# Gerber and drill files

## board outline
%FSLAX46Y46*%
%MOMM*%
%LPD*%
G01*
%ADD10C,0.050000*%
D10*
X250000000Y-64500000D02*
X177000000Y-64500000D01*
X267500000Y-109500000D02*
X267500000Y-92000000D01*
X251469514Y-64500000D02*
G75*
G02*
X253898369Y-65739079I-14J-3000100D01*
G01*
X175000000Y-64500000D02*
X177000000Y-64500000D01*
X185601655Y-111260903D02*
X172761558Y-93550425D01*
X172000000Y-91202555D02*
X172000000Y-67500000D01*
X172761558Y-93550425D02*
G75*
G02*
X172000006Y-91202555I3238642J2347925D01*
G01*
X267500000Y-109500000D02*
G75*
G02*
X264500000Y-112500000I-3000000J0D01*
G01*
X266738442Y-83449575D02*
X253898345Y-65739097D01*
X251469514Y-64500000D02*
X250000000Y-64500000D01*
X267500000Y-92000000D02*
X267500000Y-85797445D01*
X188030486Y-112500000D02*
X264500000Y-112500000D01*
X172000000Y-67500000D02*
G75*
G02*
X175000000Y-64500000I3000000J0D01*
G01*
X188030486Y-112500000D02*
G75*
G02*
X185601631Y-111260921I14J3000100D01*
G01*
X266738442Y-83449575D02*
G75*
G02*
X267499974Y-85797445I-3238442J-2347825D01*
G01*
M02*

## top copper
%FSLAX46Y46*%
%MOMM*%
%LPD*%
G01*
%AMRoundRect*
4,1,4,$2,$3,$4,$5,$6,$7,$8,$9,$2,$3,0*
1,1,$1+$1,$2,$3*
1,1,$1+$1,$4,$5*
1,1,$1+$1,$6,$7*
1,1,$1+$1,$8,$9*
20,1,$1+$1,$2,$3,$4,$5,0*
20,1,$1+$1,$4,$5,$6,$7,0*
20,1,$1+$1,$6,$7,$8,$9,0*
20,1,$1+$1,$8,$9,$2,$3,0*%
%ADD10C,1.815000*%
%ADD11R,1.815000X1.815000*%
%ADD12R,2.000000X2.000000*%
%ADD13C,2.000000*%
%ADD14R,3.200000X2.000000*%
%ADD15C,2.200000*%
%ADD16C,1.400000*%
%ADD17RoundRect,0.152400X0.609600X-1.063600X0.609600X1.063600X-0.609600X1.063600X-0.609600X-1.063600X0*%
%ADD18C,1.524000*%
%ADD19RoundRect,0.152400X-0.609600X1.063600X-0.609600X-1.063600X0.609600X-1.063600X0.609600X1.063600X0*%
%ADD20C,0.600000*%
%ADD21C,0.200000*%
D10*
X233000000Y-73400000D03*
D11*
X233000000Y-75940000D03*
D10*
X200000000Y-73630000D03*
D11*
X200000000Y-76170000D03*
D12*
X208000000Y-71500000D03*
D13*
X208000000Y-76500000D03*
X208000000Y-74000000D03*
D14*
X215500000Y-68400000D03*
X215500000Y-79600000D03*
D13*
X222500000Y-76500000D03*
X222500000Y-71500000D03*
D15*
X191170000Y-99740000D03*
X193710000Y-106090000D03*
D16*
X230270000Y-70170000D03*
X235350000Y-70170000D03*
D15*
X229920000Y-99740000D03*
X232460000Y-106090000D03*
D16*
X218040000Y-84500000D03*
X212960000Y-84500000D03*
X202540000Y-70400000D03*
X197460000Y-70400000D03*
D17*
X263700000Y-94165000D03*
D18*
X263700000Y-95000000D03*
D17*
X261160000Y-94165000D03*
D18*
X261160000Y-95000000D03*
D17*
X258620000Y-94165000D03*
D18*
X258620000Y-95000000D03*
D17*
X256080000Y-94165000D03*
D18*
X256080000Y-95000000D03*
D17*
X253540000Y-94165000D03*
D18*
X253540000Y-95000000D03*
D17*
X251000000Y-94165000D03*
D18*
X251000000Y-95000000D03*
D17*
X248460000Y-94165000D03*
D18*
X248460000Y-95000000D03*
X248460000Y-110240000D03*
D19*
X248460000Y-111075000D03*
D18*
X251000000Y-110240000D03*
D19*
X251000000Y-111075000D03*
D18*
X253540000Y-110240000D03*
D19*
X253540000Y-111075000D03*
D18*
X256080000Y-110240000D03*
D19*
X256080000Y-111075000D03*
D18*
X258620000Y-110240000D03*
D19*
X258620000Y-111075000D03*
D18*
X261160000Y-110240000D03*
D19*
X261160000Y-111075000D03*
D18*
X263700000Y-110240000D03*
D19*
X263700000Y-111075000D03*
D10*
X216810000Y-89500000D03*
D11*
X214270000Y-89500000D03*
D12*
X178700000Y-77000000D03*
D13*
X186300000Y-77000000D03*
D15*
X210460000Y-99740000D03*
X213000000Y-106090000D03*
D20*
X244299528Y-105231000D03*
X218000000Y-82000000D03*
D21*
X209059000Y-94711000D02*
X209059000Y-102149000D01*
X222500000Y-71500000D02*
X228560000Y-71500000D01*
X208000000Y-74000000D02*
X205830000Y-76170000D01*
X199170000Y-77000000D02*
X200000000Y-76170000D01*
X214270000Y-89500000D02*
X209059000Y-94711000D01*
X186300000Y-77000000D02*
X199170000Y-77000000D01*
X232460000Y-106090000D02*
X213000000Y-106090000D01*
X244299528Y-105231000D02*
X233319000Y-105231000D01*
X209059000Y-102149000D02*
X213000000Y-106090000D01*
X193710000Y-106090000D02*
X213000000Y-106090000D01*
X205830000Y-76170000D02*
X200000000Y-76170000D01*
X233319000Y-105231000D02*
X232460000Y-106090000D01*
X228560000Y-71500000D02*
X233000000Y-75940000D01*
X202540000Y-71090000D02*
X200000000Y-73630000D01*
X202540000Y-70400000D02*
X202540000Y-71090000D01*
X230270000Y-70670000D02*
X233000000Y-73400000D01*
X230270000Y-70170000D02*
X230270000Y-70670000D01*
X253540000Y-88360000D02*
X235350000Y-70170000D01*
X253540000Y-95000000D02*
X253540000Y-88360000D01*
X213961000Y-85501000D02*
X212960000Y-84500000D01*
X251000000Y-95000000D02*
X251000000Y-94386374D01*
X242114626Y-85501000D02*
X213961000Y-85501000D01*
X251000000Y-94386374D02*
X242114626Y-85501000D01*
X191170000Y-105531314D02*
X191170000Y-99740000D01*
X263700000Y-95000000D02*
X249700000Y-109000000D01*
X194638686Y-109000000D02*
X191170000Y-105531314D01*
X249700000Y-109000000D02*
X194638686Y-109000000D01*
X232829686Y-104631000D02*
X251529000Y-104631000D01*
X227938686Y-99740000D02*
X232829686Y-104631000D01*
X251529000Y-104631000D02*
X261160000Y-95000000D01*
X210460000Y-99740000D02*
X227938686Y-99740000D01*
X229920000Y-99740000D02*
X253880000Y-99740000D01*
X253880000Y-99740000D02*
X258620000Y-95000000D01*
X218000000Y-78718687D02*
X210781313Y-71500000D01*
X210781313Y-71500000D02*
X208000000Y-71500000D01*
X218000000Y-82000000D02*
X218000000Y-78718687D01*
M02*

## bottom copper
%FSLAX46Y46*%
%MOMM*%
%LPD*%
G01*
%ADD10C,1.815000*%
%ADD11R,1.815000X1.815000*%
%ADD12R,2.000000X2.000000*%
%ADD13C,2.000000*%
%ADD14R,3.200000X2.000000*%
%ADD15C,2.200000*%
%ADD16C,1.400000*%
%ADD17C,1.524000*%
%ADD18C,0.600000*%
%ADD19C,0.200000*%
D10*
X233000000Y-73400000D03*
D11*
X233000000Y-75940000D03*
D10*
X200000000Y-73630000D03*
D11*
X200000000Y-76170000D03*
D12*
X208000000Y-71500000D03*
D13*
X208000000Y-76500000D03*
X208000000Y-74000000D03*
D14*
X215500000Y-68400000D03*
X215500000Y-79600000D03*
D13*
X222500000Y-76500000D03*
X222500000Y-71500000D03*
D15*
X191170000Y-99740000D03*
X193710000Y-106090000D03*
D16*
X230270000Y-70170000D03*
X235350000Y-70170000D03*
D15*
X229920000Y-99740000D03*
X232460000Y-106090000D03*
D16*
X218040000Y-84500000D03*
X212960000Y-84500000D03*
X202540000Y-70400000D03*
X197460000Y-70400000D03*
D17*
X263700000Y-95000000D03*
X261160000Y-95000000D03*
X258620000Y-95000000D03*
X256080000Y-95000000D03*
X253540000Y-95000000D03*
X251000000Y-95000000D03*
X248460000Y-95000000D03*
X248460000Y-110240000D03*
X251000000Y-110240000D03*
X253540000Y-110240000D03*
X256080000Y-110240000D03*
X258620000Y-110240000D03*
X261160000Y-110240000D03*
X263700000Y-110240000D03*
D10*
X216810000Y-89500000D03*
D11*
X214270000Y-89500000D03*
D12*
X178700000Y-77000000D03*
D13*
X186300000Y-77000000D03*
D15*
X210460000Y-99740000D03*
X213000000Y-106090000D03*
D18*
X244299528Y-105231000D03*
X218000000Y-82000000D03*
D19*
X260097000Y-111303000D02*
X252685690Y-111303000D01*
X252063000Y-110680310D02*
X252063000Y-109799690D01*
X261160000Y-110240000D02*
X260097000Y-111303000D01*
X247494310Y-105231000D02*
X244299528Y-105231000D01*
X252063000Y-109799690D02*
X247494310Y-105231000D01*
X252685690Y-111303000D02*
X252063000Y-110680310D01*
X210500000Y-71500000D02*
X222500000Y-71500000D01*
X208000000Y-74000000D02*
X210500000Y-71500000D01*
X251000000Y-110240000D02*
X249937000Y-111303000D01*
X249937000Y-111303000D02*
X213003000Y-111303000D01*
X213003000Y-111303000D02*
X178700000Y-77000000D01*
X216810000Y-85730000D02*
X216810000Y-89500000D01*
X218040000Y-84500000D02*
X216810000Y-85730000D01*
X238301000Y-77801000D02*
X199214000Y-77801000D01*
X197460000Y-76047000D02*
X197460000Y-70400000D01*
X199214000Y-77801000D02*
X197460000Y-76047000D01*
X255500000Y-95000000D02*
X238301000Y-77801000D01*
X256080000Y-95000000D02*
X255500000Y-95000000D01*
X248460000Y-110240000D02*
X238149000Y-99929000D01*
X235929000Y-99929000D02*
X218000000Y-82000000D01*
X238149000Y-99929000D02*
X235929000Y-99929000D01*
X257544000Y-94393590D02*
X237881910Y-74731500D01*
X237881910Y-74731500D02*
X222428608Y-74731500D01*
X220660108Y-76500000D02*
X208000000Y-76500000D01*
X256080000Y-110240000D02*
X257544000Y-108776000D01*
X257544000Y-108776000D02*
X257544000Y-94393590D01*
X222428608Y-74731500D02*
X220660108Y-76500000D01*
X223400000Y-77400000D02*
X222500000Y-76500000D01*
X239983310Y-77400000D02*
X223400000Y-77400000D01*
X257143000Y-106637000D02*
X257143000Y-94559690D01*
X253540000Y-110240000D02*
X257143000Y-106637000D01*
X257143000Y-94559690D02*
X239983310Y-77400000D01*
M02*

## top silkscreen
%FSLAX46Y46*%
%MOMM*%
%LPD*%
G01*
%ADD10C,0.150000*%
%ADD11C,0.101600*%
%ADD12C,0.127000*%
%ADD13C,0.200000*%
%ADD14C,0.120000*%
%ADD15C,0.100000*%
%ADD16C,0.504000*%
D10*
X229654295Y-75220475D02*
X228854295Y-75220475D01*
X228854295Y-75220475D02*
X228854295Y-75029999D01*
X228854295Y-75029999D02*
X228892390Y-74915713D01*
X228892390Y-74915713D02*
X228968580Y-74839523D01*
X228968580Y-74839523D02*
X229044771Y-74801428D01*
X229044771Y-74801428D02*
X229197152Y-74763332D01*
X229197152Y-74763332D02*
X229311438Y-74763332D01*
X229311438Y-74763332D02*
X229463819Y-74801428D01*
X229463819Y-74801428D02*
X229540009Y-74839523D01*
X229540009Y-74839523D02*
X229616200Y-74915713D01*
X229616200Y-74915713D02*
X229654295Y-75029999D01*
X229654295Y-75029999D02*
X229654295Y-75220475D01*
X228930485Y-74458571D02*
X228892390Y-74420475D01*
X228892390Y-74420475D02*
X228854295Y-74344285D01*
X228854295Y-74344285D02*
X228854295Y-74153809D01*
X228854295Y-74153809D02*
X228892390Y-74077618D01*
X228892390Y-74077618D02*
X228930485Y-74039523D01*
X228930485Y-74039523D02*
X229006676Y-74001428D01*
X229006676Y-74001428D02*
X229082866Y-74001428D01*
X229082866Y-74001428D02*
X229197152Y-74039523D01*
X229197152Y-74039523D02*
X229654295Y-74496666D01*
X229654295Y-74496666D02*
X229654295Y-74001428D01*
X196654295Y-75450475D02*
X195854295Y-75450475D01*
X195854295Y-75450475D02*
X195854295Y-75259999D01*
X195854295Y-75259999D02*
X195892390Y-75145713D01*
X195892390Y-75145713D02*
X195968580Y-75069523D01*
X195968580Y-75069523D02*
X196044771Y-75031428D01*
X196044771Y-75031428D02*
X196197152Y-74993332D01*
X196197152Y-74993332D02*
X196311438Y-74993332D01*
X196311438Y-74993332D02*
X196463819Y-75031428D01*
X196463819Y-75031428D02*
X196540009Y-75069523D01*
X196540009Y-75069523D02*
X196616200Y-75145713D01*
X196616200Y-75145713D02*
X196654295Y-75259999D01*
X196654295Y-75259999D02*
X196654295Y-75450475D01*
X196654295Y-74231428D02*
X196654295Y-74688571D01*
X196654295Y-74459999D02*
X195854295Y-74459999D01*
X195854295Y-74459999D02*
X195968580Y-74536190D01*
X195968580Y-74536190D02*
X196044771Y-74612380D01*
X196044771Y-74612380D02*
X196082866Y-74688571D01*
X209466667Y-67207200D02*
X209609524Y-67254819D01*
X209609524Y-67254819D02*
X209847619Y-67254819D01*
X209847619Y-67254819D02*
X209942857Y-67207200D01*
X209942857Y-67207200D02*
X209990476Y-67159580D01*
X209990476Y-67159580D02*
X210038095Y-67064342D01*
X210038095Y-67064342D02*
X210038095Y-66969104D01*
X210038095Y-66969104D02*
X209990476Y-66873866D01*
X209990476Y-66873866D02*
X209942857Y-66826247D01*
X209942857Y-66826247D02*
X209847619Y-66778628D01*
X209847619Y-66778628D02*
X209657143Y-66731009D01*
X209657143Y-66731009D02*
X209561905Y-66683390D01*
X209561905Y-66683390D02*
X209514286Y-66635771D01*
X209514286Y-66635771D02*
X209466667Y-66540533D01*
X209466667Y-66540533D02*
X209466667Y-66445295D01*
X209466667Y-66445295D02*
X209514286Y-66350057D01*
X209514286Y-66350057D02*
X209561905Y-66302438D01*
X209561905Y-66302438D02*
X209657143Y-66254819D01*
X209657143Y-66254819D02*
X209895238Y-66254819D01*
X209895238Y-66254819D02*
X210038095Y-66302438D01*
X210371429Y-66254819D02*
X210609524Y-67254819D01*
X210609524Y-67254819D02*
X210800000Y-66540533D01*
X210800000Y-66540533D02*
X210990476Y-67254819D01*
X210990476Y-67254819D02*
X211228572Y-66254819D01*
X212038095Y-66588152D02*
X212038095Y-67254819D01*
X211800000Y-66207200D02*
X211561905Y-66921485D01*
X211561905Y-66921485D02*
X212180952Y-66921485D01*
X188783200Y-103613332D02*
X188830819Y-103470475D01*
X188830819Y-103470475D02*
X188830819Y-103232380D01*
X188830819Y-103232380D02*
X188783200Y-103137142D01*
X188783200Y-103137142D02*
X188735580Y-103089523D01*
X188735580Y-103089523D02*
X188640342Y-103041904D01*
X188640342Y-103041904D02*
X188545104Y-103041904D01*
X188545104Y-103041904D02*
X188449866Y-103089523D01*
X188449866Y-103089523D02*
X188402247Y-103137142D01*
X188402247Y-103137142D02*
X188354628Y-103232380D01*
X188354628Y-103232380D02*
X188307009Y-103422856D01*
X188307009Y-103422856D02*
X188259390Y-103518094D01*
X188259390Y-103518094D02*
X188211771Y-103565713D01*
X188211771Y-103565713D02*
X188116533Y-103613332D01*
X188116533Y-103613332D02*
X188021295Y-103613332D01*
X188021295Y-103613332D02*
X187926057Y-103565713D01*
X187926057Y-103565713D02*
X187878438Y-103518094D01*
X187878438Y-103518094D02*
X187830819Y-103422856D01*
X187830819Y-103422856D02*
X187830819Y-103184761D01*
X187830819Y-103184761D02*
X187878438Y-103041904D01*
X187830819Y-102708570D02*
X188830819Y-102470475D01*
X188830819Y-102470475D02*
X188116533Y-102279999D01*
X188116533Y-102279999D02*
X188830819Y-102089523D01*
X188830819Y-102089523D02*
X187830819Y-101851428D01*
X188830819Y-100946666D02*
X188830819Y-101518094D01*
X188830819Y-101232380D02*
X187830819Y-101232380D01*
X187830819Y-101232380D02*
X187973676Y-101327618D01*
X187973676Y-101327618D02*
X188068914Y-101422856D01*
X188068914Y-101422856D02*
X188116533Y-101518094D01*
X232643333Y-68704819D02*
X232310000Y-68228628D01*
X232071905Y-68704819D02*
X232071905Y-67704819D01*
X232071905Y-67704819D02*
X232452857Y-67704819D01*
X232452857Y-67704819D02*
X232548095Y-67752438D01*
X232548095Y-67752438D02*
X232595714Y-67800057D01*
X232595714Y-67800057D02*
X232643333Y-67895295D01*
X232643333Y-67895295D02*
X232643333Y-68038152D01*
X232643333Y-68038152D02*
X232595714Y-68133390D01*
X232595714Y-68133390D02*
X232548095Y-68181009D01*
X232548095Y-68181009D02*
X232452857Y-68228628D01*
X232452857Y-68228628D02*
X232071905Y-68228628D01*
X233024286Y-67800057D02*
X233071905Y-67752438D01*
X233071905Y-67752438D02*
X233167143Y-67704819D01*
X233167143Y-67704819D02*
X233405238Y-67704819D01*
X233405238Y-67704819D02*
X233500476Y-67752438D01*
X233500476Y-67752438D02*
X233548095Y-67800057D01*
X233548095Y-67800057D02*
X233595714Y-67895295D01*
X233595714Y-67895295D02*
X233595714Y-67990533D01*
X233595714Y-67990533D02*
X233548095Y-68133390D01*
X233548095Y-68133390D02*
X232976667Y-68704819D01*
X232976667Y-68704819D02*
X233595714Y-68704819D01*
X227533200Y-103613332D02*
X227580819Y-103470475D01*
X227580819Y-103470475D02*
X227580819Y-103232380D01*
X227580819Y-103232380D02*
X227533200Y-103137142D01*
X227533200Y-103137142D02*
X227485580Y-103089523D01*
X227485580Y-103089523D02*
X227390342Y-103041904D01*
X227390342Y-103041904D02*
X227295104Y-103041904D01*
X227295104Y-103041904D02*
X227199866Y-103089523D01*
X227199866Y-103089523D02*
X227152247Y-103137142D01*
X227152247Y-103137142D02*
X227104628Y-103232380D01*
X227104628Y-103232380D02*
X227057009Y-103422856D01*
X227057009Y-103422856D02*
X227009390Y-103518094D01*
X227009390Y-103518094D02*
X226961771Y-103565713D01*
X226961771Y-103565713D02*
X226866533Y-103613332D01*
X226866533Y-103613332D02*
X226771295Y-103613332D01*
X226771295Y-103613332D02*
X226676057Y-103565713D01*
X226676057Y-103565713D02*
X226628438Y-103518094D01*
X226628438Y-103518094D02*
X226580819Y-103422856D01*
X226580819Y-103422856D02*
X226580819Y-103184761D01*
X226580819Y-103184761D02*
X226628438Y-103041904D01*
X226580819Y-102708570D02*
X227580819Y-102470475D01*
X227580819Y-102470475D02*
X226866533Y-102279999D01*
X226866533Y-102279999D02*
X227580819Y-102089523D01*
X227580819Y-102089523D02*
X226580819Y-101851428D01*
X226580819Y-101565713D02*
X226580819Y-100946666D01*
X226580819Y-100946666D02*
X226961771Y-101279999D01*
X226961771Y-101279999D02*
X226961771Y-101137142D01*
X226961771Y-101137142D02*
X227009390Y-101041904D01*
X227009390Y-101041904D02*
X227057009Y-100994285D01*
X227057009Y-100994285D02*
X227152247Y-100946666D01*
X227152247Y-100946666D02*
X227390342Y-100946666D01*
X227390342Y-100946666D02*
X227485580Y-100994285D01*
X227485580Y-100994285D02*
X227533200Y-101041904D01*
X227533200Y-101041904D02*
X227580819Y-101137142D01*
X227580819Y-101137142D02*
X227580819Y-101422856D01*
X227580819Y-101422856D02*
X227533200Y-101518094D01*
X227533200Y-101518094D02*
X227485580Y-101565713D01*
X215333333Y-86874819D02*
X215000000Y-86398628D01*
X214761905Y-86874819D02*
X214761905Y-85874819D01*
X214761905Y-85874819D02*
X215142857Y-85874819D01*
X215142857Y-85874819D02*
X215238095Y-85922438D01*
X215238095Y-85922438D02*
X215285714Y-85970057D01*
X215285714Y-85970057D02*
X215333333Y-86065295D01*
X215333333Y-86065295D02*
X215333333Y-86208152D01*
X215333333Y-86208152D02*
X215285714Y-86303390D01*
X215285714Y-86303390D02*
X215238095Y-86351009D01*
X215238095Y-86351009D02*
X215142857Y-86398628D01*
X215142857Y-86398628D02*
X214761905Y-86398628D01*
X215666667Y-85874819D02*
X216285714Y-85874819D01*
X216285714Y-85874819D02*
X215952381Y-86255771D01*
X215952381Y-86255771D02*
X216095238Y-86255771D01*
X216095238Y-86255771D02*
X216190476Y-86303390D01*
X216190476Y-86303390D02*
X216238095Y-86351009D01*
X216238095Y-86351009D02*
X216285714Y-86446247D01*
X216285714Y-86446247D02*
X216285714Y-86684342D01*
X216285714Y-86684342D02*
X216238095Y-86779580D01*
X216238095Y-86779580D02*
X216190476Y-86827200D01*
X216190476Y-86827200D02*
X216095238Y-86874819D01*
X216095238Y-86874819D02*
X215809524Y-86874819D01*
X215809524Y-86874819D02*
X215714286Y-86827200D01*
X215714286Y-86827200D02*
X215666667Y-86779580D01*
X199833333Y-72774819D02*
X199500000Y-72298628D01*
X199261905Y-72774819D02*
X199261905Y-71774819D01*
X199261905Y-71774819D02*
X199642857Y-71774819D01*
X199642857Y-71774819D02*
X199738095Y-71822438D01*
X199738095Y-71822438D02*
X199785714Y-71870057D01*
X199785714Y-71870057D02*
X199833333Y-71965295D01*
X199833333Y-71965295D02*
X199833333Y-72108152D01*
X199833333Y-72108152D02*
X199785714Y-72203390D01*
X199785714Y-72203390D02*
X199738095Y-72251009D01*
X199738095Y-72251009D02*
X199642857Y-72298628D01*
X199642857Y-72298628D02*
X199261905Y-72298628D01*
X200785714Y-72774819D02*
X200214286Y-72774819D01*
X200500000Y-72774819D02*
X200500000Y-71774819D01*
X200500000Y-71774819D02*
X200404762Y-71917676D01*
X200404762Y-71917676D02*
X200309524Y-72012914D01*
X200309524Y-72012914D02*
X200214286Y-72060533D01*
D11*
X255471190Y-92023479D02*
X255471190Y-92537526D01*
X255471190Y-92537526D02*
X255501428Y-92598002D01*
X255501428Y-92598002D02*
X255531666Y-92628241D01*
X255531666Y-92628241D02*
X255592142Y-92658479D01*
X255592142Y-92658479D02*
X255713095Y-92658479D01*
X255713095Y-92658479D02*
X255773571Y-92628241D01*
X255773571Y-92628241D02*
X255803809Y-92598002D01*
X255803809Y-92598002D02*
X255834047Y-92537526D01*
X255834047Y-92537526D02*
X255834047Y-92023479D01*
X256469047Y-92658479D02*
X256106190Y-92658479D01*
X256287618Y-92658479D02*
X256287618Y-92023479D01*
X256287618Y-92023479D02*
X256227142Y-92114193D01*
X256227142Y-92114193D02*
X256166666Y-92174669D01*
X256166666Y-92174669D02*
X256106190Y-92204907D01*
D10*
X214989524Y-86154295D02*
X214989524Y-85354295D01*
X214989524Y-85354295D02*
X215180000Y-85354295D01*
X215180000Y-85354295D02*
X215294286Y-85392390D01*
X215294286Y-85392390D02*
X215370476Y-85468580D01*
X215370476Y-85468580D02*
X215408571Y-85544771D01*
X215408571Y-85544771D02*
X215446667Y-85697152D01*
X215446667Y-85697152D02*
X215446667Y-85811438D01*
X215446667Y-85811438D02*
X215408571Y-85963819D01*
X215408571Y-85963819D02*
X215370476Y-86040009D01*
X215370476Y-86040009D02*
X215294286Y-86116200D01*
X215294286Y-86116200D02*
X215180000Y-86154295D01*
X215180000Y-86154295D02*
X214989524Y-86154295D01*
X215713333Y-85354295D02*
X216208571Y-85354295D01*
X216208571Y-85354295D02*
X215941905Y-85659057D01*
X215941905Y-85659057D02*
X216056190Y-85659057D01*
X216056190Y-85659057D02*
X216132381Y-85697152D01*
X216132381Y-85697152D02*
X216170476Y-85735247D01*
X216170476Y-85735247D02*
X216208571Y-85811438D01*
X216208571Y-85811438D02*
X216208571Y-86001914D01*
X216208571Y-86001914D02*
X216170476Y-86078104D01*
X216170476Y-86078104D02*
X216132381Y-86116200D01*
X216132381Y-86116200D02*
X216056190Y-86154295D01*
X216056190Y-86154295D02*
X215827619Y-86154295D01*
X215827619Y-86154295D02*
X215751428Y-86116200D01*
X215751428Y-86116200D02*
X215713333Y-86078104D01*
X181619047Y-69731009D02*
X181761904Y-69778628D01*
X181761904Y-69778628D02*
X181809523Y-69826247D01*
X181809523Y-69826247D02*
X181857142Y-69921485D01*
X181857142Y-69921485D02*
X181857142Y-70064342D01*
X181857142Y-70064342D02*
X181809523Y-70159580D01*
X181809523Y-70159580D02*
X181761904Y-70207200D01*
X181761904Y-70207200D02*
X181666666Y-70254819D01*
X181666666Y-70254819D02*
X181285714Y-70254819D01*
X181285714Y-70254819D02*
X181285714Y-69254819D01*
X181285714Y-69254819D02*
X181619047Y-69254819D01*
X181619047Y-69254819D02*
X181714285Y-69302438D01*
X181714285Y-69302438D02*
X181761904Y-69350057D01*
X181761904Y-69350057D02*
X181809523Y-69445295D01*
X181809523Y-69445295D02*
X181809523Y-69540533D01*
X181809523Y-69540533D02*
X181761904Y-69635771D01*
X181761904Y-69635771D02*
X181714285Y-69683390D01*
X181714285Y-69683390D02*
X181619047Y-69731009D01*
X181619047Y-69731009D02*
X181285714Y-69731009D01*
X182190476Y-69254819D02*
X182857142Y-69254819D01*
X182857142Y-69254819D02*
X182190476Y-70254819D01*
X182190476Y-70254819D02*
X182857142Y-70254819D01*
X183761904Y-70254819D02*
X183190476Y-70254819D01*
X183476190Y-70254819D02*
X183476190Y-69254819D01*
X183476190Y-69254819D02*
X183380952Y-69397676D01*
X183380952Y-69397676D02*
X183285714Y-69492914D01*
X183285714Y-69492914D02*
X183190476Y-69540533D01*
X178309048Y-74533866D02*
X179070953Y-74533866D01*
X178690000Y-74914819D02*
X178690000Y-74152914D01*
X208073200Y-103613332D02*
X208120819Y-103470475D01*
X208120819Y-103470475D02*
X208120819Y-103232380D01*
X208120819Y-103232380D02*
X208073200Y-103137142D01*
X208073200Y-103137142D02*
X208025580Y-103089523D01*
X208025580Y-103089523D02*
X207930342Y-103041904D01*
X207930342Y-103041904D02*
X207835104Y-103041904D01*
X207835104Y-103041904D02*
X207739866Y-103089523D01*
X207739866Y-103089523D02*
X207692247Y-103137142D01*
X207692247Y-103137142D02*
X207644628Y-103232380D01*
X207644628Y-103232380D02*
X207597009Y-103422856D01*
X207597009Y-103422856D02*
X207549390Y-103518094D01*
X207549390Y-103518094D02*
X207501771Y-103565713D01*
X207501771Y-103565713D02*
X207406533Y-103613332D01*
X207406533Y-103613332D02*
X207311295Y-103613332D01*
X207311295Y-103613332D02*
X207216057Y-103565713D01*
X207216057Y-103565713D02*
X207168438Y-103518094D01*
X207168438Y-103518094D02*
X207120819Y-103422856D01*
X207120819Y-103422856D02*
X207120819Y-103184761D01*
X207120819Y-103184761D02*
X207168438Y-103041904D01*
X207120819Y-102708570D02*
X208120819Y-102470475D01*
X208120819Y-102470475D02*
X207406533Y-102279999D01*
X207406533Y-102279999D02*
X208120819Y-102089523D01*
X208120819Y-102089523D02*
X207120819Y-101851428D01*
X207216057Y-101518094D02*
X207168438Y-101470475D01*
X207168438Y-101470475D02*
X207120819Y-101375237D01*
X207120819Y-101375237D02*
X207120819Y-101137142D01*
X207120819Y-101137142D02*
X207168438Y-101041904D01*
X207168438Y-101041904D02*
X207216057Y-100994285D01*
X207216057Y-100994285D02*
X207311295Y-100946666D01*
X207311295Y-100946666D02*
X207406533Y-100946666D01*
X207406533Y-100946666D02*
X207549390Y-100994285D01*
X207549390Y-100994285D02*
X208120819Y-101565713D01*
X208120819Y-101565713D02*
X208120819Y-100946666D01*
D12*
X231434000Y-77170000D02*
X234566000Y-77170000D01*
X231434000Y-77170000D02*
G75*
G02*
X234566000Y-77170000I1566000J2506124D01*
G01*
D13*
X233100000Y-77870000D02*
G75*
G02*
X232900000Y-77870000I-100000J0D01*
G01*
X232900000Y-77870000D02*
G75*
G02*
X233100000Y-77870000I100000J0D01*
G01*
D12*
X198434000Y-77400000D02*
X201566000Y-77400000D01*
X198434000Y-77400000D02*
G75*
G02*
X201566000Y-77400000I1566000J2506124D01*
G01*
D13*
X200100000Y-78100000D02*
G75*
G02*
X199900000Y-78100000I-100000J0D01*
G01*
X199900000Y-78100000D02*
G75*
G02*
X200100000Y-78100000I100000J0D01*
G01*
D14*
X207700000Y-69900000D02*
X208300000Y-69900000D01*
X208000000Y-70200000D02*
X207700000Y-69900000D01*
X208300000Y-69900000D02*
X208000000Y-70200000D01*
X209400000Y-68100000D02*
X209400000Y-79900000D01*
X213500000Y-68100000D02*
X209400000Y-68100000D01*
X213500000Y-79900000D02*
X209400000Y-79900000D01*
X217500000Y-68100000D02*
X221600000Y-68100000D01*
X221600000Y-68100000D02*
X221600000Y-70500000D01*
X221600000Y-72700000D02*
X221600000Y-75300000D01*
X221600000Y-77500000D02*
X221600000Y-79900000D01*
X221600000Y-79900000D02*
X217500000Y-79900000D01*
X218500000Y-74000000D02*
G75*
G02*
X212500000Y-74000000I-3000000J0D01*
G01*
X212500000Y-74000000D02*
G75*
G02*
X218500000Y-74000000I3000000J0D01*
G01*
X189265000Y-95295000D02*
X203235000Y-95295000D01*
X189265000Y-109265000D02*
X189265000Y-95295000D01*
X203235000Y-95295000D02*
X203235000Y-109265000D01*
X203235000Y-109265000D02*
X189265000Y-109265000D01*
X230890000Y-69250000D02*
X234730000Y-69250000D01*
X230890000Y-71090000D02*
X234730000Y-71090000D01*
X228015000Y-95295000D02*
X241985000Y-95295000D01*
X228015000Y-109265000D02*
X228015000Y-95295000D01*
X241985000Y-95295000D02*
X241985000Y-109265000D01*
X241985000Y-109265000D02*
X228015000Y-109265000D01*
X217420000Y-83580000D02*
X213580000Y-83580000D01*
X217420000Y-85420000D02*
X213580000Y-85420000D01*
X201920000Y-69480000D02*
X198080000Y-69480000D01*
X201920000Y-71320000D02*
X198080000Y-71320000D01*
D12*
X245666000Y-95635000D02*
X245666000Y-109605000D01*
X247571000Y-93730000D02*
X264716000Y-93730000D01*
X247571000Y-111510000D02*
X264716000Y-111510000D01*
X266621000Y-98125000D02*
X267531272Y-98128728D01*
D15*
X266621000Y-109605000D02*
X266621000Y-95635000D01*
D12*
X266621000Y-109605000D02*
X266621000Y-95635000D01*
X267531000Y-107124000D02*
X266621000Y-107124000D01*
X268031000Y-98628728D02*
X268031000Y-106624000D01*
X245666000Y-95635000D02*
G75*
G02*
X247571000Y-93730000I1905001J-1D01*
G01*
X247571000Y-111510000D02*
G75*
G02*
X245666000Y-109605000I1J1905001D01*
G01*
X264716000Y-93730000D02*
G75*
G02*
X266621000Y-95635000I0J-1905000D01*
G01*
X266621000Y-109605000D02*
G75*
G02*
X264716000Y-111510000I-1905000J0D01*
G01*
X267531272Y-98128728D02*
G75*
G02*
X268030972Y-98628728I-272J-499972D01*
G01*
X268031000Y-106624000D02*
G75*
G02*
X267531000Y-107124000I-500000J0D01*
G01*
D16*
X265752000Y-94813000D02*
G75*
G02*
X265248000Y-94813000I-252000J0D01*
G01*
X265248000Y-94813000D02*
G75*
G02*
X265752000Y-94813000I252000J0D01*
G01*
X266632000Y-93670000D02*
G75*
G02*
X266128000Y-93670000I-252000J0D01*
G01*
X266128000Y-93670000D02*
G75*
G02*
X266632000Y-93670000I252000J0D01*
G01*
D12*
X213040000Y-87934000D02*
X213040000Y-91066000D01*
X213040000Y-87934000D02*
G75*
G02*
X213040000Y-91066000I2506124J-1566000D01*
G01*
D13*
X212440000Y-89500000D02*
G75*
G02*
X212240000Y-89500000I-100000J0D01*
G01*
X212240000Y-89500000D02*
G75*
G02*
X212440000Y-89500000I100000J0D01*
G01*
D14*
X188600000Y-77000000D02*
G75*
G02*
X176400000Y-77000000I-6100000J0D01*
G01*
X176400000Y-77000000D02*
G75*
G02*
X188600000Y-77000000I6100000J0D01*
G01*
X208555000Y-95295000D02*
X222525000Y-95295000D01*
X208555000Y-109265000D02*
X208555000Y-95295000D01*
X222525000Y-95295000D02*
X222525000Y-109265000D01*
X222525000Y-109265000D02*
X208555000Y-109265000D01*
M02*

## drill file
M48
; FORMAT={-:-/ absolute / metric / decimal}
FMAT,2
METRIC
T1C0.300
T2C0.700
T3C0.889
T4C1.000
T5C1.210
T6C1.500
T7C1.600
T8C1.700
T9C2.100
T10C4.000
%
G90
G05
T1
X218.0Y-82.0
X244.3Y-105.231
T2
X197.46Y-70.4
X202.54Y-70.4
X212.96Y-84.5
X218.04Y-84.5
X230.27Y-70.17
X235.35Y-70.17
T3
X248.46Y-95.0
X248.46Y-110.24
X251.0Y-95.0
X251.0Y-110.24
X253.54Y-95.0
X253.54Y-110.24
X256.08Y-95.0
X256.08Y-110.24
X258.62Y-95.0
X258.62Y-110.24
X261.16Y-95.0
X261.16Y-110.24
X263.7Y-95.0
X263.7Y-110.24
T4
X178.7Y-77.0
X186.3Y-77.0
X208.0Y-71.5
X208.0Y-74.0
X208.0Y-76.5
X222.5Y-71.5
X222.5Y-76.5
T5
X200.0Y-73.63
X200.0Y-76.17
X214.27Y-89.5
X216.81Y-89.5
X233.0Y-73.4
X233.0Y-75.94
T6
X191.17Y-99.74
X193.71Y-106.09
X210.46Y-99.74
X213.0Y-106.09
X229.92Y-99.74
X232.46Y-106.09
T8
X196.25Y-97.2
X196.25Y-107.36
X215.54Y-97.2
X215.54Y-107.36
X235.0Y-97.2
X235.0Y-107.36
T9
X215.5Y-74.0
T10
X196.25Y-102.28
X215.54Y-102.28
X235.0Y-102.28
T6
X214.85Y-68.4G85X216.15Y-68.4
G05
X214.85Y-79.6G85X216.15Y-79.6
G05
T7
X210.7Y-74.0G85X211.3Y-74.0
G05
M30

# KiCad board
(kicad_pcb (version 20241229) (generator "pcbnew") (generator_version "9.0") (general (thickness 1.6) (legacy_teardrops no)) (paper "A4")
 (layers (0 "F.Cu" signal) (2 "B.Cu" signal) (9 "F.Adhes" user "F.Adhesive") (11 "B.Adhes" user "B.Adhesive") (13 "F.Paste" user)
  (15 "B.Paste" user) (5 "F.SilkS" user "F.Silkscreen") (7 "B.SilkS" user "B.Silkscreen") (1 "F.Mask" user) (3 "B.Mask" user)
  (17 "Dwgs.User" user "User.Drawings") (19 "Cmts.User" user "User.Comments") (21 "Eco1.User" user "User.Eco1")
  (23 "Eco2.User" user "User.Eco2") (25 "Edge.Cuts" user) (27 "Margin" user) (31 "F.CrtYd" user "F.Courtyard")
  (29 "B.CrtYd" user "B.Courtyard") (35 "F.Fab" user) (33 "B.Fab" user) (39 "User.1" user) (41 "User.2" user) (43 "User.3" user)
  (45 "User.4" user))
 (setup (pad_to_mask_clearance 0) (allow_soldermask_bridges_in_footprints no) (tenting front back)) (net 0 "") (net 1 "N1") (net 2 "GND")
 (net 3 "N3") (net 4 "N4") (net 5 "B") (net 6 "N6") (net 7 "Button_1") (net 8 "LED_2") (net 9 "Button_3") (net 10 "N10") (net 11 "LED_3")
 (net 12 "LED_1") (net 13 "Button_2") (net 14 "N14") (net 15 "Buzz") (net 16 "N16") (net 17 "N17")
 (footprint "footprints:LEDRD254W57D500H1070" (layer "F.Cu") (at 233 74.67 90)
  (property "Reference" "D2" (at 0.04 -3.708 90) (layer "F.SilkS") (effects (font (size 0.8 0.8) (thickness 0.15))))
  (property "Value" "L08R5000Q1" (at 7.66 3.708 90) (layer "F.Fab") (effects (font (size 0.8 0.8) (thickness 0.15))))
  (fp_line (start -2.5 -1.566) (end -2.5 1.566) (stroke (width 0.127) (type solid)) (layer "F.SilkS"))
  (fp_arc (start -2.5 -1.566) (mid 2.961291 0) (end -2.5 1.566) (stroke (width 0.127) (type solid)) (layer "F.SilkS"))
  (fp_circle (center -3.2 0) (end -3.1 0) (stroke (width 0.2) (type solid)) (fill no) (layer "F.SilkS"))
  (pad "A" thru_hole circle (at 1.27 0 90) (size 1.815 1.815) (drill 1.21) (layers "*.Cu" "*.Mask") (remove_unused_layers no) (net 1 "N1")
   (solder_mask_margin 0.102))
  (pad "C" thru_hole rect (at -1.27 0 90) (size 1.815 1.815) (drill 1.21) (layers "*.Cu" "*.Mask") (remove_unused_layers no) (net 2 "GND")
   (solder_mask_margin 0.102)))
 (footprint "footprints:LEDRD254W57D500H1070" (layer "F.Cu") (at 200 74.9 90)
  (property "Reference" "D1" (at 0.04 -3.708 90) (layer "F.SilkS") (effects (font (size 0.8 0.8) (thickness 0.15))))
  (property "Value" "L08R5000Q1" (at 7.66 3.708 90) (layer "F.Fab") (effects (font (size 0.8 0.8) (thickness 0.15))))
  (fp_line (start -2.5 -1.566) (end -2.5 1.566) (stroke (width 0.127) (type solid)) (layer "F.SilkS"))
  (fp_arc (start -2.5 -1.566) (mid 2.961291 0) (end -2.5 1.566) (stroke (width 0.127) (type solid)) (layer "F.SilkS"))
  (fp_circle (center -3.2 0) (end -3.1 0) (stroke (width 0.2) (type solid)) (fill no) (layer "F.SilkS"))
  (pad "A" thru_hole circle (at 1.27 0 90) (size 1.815 1.815) (drill 1.21) (layers "*.Cu" "*.Mask") (remove_unused_layers no) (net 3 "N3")
   (solder_mask_margin 0.102))
  (pad "C" thru_hole rect (at -1.27 0 90) (size 1.815 1.815) (drill 1.21) (layers "*.Cu" "*.Mask") (remove_unused_layers no) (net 2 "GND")
   (solder_mask_margin 0.102)))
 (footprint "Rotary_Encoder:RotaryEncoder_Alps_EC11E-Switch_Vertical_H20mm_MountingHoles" (layer "F.Cu") (at 208 71.5)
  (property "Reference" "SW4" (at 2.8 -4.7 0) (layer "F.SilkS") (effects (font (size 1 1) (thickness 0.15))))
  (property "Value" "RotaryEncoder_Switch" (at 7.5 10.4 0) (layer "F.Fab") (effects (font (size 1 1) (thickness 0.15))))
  (fp_line (start -0.3 -1.6) (end 0.3 -1.6) (stroke (width 0.12) (type solid)) (layer "F.SilkS"))
  (fp_line (start 0 -1.3) (end -0.3 -1.6) (stroke (width 0.12) (type solid)) (layer "F.SilkS"))
  (fp_line (start 0.3 -1.6) (end 0 -1.3) (stroke (width 0.12) (type solid)) (layer "F.SilkS"))
  (fp_line (start 1.4 -3.4) (end 1.4 8.4) (stroke (width 0.12) (type solid)) (layer "F.SilkS"))
  (fp_line (start 5.5 -3.4) (end 1.4 -3.4) (stroke (width 0.12) (type solid)) (layer "F.SilkS"))
  (fp_line (start 5.5 8.4) (end 1.4 8.4) (stroke (width 0.12) (type solid)) (layer "F.SilkS"))
  (fp_line (start 9.5 -3.4) (end 13.6 -3.4) (stroke (width 0.12) (type solid)) (layer "F.SilkS"))
  (fp_line (start 13.6 -3.4) (end 13.6 -1) (stroke (width 0.12) (type solid)) (layer "F.SilkS"))
  (fp_line (start 13.6 1.2) (end 13.6 3.8) (stroke (width 0.12) (type solid)) (layer "F.SilkS"))
  (fp_line (start 13.6 6) (end 13.6 8.4) (stroke (width 0.12) (type solid)) (layer "F.SilkS"))
  (fp_line (start 13.6 8.4) (end 9.5 8.4) (stroke (width 0.12) (type solid)) (layer "F.SilkS"))
  (fp_circle (center 7.5 2.5) (end 10.5 2.5) (stroke (width 0.12) (type solid)) (fill no) (layer "F.SilkS"))
  (pad "" np_thru_hole oval (at 3 2.5) (size 2.2 1.6) (drill oval 2.2 1.6) (layers "*.Mask"))
  (pad "" np_thru_hole circle (at 7.5 2.5) (size 2.1 2.1) (drill 2.1) (layers "*.Mask"))
  (pad "A" thru_hole rect (at 0 0) (size 2 2) (drill 1) (layers "*.Cu" "*.Mask") (remove_unused_layers no) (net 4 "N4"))
  (pad "B" thru_hole circle (at 0 5) (size 2 2) (drill 1) (layers "*.Cu" "*.Mask") (remove_unused_layers no) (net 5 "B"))
  (pad "C" thru_hole circle (at 0 2.5) (size 2 2) (drill 1) (layers "*.Cu" "*.Mask") (remove_unused_layers no) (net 2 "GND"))
  (pad "MP" thru_hole rect (at 7.5 -3.1) (size 3.2 2) (drill oval 2.8 1.5) (layers "*.Cu" "*.Mask") (remove_unused_layers no))
  (pad "MP" thru_hole rect (at 7.5 8.1) (size 3.2 2) (drill oval 2.8 1.5) (layers "*.Cu" "*.Mask") (remove_unused_layers no))
  (pad "S1" thru_hole circle (at 14.5 5) (size 2 2) (drill 1) (layers "*.Cu" "*.Mask") (remove_unused_layers no) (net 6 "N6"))
  (pad "S2" thru_hole circle (at 14.5 0) (size 2 2) (drill 1) (layers "*.Cu" "*.Mask") (remove_unused_layers no) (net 2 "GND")))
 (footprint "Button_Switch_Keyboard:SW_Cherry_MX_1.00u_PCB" (layer "F.Cu") (at 191.17 99.74 90)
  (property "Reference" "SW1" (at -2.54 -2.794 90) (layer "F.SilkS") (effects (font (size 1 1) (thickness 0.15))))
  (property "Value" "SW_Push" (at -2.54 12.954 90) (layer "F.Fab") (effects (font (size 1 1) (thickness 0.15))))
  (fp_line (start 4.445 -1.905) (end 4.445 12.065) (stroke (width 0.12) (type solid)) (layer "F.SilkS"))
  (fp_line (start -9.525 -1.905) (end 4.445 -1.905) (stroke (width 0.12) (type solid)) (layer "F.SilkS"))
  (fp_line (start 4.445 12.065) (end -9.525 12.065) (stroke (width 0.12) (type solid)) (layer "F.SilkS"))
  (fp_line (start -9.525 12.065) (end -9.525 -1.905) (stroke (width 0.12) (type solid)) (layer "F.SilkS"))
  (pad "" np_thru_hole circle (at -7.62 5.08 90) (size 1.7 1.7) (drill 1.7) (layers "*.Cu" "*.Mask"))
  (pad "" np_thru_hole circle (at -2.54 5.08 90) (size 4 4) (drill 4) (layers "*.Cu" "*.Mask"))
  (pad "" np_thru_hole circle (at 2.54 5.08 90) (size 1.7 1.7) (drill 1.7) (layers "*.Cu" "*.Mask"))
  (pad "1" thru_hole circle (at 0 0 90) (size 2.2 2.2) (drill 1.5) (layers "*.Cu" "*.Mask") (remove_unused_layers no) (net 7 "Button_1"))
  (pad "2" thru_hole circle (at -6.35 2.54 90) (size 2.2 2.2) (drill 1.5) (layers "*.Cu" "*.Mask") (remove_unused_layers no) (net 2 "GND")))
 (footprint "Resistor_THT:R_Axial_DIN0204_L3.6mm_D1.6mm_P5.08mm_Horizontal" (layer "F.Cu") (at 230.27 70.17)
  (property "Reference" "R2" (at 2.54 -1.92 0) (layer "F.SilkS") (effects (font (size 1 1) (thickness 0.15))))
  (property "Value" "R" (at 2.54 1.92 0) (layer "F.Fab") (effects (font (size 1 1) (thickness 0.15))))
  (fp_line (start 0.62 -0.92) (end 4.46 -0.92) (stroke (width 0.12) (type solid)) (layer "F.SilkS"))
  (fp_line (start 0.62 0.92) (end 4.46 0.92) (stroke (width 0.12) (type solid)) (layer "F.SilkS"))
  (pad "1" thru_hole circle (at 0 0) (size 1.4 1.4) (drill 0.7) (layers "*.Cu" "*.Mask") (remove_unused_layers no) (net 1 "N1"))
  (pad "2" thru_hole circle (at 5.08 0) (size 1.4 1.4) (drill 0.7) (layers "*.Cu" "*.Mask") (remove_unused_layers no) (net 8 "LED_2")))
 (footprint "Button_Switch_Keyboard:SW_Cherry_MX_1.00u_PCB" (layer "F.Cu") (at 229.92 99.74 90)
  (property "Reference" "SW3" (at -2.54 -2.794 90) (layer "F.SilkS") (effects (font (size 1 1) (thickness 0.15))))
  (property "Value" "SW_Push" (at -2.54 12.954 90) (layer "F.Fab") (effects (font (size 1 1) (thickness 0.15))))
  (fp_line (start 4.445 -1.905) (end 4.445 12.065) (stroke (width 0.12) (type solid)) (layer "F.SilkS"))
  (fp_line (start -9.525 -1.905) (end 4.445 -1.905) (stroke (width 0.12) (type solid)) (layer "F.SilkS"))
  (fp_line (start 4.445 12.065) (end -9.525 12.065) (stroke (width 0.12) (type solid)) (layer "F.SilkS"))
  (fp_line (start -9.525 12.065) (end -9.525 -1.905) (stroke (width 0.12) (type solid)) (layer "F.SilkS"))
  (pad "" np_thru_hole circle (at -7.62 5.08 90) (size 1.7 1.7) (drill 1.7) (layers "*.Cu" "*.Mask"))
  (pad "" np_thru_hole circle (at -2.54 5.08 90) (size 4 4) (drill 4) (layers "*.Cu" "*.Mask"))
  (pad "" np_thru_hole circle (at 2.54 5.08 90) (size 1.7 1.7) (drill 1.7) (layers "*.Cu" "*.Mask"))
  (pad "1" thru_hole circle (at 0 0 90) (size 2.2 2.2) (drill 1.5) (layers "*.Cu" "*.Mask") (remove_unused_layers no) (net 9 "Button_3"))
  (pad "2" thru_hole circle (at -6.35 2.54 90) (size 2.2 2.2) (drill 1.5) (layers "*.Cu" "*.Mask") (remove_unused_layers no) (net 2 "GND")))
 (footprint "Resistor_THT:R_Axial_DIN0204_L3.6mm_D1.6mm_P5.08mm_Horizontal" (layer "F.Cu") (at 218.04 84.5 180)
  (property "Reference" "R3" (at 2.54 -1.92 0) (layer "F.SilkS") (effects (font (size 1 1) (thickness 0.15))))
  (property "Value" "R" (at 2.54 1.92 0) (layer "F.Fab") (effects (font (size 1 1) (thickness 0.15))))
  (fp_line (start 0.62 0.92) (end 4.46 0.92) (stroke (width 0.12) (type solid)) (layer "F.SilkS"))
  (fp_line (start 0.62 -0.92) (end 4.46 -0.92) (stroke (width 0.12) (type solid)) (layer "F.SilkS"))
  (pad "1" thru_hole circle (at 0 0 180) (size 1.4 1.4) (drill 0.7) (layers "*.Cu" "*.Mask") (remove_unused_layers no) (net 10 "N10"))
  (pad "2" thru_hole circle (at 5.08 0 180) (size 1.4 1.4) (drill 0.7) (layers "*.Cu" "*.Mask") (remove_unused_layers no) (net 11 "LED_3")))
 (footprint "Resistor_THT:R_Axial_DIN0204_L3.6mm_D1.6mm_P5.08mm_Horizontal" (layer "F.Cu") (at 202.54 70.4 180)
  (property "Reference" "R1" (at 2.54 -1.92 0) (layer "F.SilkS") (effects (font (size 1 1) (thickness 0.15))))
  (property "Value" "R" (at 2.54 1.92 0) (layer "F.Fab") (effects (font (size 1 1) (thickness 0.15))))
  (fp_line (start 0.62 0.92) (end 4.46 0.92) (stroke (width 0.12) (type solid)) (layer "F.SilkS"))
  (fp_line (start 0.62 -0.92) (end 4.46 -0.92) (stroke (width 0.12) (type solid)) (layer "F.SilkS"))
  (pad "1" thru_hole circle (at 0 0 180) (size 1.4 1.4) (drill 0.7) (layers "*.Cu" "*.Mask") (remove_unused_layers no) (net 3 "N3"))
  (pad "2" thru_hole circle (at 5.08 0 180) (size 1.4 1.4) (drill 0.7) (layers "*.Cu" "*.Mask") (remove_unused_layers no) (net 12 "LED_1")))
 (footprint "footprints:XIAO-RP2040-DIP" (layer "F.Cu") (at 256.08 102.62)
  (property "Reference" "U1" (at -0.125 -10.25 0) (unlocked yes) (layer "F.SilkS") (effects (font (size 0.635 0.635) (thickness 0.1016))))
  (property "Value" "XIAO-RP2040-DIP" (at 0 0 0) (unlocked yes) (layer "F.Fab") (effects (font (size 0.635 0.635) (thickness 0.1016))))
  (fp_line (start -10.414 -6.985) (end -10.414 6.985) (stroke (width 0.127) (type solid)) (layer "F.SilkS"))
  (fp_line (start -8.509 -8.89) (end 8.636 -8.89) (stroke (width 0.127) (type solid)) (layer "F.SilkS"))
  (fp_line (start -8.509 8.89) (end 8.636 8.89) (stroke (width 0.127) (type solid)) (layer "F.SilkS"))
  (fp_line (start 10.541 -4.495) (end 11.451272 -4.491272) (stroke (width 0.127) (type solid)) (layer "F.SilkS"))
  (fp_line (start 10.541 6.985) (end 10.541 -6.985) (stroke (width 0.1) (type solid)) (layer "F.SilkS"))
  (fp_line (start 10.541 6.985) (end 10.541 -6.985) (stroke (width 0.127) (type solid)) (layer "F.SilkS"))
  (fp_line (start 11.451 4.504) (end 10.541 4.504) (stroke (width 0.127) (type solid)) (layer "F.SilkS"))
  (fp_line (start 11.951 -3.991272) (end 11.951 4.004) (stroke (width 0.127) (type solid)) (layer "F.SilkS"))
  (fp_arc (start -10.414 -6.985) (mid -9.856038 -8.332038) (end -8.509 -8.89) (stroke (width 0.127) (type solid)) (layer "F.SilkS"))
  (fp_arc (start -8.509 8.89) (mid -9.856038 8.332038) (end -10.414 6.985) (stroke (width 0.127) (type solid)) (layer "F.SilkS"))
  (fp_arc (start 8.636 -8.89) (mid 9.983038 -8.332038) (end 10.541 -6.985) (stroke (width 0.127) (type solid)) (layer "F.SilkS"))
  (fp_arc (start 10.541 6.985) (mid 9.983038 8.332038) (end 8.636 8.89) (stroke (width 0.127) (type solid)) (layer "F.SilkS"))
  (fp_arc (start 11.451272 -4.491272) (mid 11.804644 -4.344724) (end 11.951 -3.991272) (stroke (width 0.127) (type default))
   (layer "F.SilkS"))
  (fp_arc (start 11.951 4.004) (mid 11.804553 4.357553) (end 11.451 4.504) (stroke (width 0.127) (type default)) (layer "F.SilkS"))
  (fp_circle (center 9.42 -7.807) (end 9.674 -7.807) (stroke (width 0.5) (type solid)) (fill yes) (layer "F.SilkS"))
  (fp_circle (center 10.3 -8.95) (end 10.554 -8.95) (stroke (width 0.5) (type solid)) (fill yes) (layer "F.SilkS"))
  (pad "1" smd roundrect (at 7.62 -8.455 90) (size 2.432 1.524) (layers "F.Cu" "F.Mask") (roundrect_rratio 0.1) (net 7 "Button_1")
   (thermal_bridge_angle 45))
  (pad "1" thru_hole circle (at 7.62 -7.62 90) (size 1.524 1.524) (drill 0.889) (layers "*.Cu" "*.Mask") (remove_unused_layers no)
   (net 7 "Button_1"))
  (pad "2" smd roundrect (at 5.08 -8.455 90) (size 2.432 1.524) (layers "F.Cu" "F.Mask") (roundrect_rratio 0.1) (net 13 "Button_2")
   (thermal_bridge_angle 45))
  (pad "2" thru_hole circle (at 5.08 -7.62 90) (size 1.524 1.524) (drill 0.889) (layers "*.Cu" "*.Mask") (remove_unused_layers no)
   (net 13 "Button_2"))
  (pad "3" smd roundrect (at 2.54 -8.455 90) (size 2.432 1.524) (layers "F.Cu" "F.Mask") (roundrect_rratio 0.1) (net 9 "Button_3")
   (thermal_bridge_angle 45))
  (pad "3" thru_hole circle (at 2.54 -7.62 90) (size 1.524 1.524) (drill 0.889) (layers "*.Cu" "*.Mask") (remove_unused_layers no)
   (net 9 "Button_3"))
  (pad "4" smd roundrect (at 0 -8.455 90) (size 2.432 1.524) (layers "F.Cu" "F.Mask") (roundrect_rratio 0.1) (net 12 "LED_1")
   (thermal_bridge_angle 45))
  (pad "4" thru_hole circle (at 0 -7.62 90) (size 1.524 1.524) (drill 0.889) (layers "*.Cu" "*.Mask") (remove_unused_layers no)
   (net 12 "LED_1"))
  (pad "5" smd roundrect (at -2.54 -8.455 90) (size 2.432 1.524) (layers "F.Cu" "F.Mask") (roundrect_rratio 0.1) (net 8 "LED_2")
   (thermal_bridge_angle 45))
  (pad "5" thru_hole circle (at -2.54 -7.62 90) (size 1.524 1.524) (drill 0.889) (layers "*.Cu" "*.Mask") (remove_unused_layers no)
   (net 8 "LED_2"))
  (pad "6" smd roundrect (at -5.08 -8.455 90) (size 2.432 1.524) (layers "F.Cu" "F.Mask") (roundrect_rratio 0.1) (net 11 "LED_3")
   (thermal_bridge_angle 45))
  (pad "6" thru_hole circle (at -5.08 -7.62 90) (size 1.524 1.524) (drill 0.889) (layers "*.Cu" "*.Mask") (remove_unused_layers no)
   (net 11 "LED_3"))
  (pad "7" smd roundrect (at -7.62 -8.455 90) (size 2.432 1.524) (layers "F.Cu" "F.Mask") (roundrect_rratio 0.1) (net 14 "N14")
   (thermal_bridge_angle 45))
  (pad "7" thru_hole circle (at -7.62 -7.62 90) (size 1.524 1.524) (drill 0.889) (layers "*.Cu" "*.Mask") (remove_unused_layers no)
   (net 14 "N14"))
  (pad "8" thru_hole circle (at -7.62 7.62 270) (size 1.524 1.524) (drill 0.889) (layers "*.Cu" "*.Mask") (remove_unused_layers no)
   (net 4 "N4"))
  (pad "8" smd roundrect (at -7.62 8.455 270) (size 2.432 1.524) (layers "F.Cu" "F.Mask") (roundrect_rratio 0.1) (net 4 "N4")
   (thermal_bridge_angle 45))
  (pad "9" thru_hole circle (at -5.08 7.62 270) (size 1.524 1.524) (drill 0.889) (layers "*.Cu" "*.Mask") (remove_unused_layers no)
   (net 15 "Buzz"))
  (pad "9" smd roundrect (at -5.08 8.455 270) (size 2.432 1.524) (layers "F.Cu" "F.Mask") (roundrect_rratio 0.1) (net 15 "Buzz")
   (thermal_bridge_angle 45))
  (pad "10" thru_hole circle (at -2.54 7.62 270) (size 1.524 1.524) (drill 0.889) (layers "*.Cu" "*.Mask") (remove_unused_layers no)
   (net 6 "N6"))
  (pad "10" smd roundrect (at -2.54 8.455 270) (size 2.432 1.524) (layers "F.Cu" "F.Mask") (roundrect_rratio 0.1) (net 6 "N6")
   (thermal_bridge_angle 45))
  (pad "11" thru_hole circle (at 0 7.62 270) (size 1.524 1.524) (drill 0.889) (layers "*.Cu" "*.Mask") (remove_unused_layers no) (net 5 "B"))
  (pad "11" smd roundrect (at 0 8.455 270) (size 2.432 1.524) (layers "F.Cu" "F.Mask") (roundrect_rratio 0.1) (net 5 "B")
   (thermal_bridge_angle 45))
  (pad "12" thru_hole circle (at 2.54 7.62 270) (size 1.524 1.524) (drill 0.889) (layers "*.Cu" "*.Mask") (remove_unused_layers no)
   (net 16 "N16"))
  (pad "12" smd roundrect (at 2.54 8.455 270) (size 2.432 1.524) (layers "F.Cu" "F.Mask") (roundrect_rratio 0.1) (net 16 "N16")
   (thermal_bridge_angle 45))
  (pad "13" thru_hole circle (at 5.08 7.62 270) (size 1.524 1.524) (drill 0.889) (layers "*.Cu" "*.Mask") (remove_unused_layers no)
   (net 2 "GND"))
  (pad "13" smd roundrect (at 5.08 8.455 270) (size 2.432 1.524) (layers "F.Cu" "F.Mask") (roundrect_rratio 0.1) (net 2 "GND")
   (thermal_bridge_angle 45))
  (pad "14" thru_hole circle (at 7.62 7.62 270) (size 1.524 1.524) (drill 0.889) (layers "*.Cu" "*.Mask") (remove_unused_layers no)
   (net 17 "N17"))
  (pad "14" smd roundrect (at 7.62 8.455 270) (size 2.432 1.524) (layers "F.Cu" "F.Mask") (roundrect_rratio 0.1) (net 17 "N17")
   (thermal_bridge_angle 45)))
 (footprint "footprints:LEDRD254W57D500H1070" (layer "F.Cu") (at 215.54 89.5)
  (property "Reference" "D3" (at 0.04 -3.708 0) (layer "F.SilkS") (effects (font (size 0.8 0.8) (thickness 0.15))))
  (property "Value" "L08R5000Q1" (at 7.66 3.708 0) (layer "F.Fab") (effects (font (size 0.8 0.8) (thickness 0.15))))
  (fp_line (start -2.5 -1.566) (end -2.5 1.566) (stroke (width 0.127) (type solid)) (layer "F.SilkS"))
  (fp_arc (start -2.5 -1.566) (mid 2.961291 0) (end -2.5 1.566) (stroke (width 0.127) (type solid)) (layer "F.SilkS"))
  (fp_circle (center -3.2 0) (end -3.1 0) (stroke (width 0.2) (type solid)) (fill no) (layer "F.SilkS"))
  (pad "A" thru_hole circle (at 1.27 0) (size 1.815 1.815) (drill 1.21) (layers "*.Cu" "*.Mask") (remove_unused_layers no) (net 10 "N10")
   (solder_mask_margin 0.102))
  (pad "C" thru_hole rect (at -1.27 0) (size 1.815 1.815) (drill 1.21) (layers "*.Cu" "*.Mask") (remove_unused_layers no) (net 2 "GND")
   (solder_mask_margin 0.102)))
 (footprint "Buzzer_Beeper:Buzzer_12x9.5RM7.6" (layer "F.Cu") (at 178.7 77)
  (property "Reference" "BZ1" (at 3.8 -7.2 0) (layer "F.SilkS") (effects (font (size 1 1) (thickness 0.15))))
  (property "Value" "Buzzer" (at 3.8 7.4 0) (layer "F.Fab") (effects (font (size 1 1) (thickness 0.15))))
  (fp_circle (center 3.8 0) (end 9.9 0) (stroke (width 0.12) (type solid)) (fill no) (layer "F.SilkS"))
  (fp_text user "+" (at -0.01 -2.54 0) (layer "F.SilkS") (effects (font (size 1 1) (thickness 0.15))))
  (pad "1" thru_hole rect (at 0 0) (size 2 2) (drill 1) (layers "*.Cu" "*.Mask") (remove_unused_layers no) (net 15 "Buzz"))
  (pad "2" thru_hole circle (at 7.6 0) (size 2 2) (drill 1) (layers "*.Cu" "*.Mask") (remove_unused_layers no) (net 2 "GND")))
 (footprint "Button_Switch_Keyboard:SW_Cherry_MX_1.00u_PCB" (layer "F.Cu") (at 210.46 99.74 90)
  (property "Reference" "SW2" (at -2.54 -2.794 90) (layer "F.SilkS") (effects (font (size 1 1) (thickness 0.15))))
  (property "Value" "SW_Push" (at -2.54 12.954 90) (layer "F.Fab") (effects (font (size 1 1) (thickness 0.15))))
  (fp_line (start 4.445 -1.905) (end 4.445 12.065) (stroke (width 0.12) (type solid)) (layer "F.SilkS"))
  (fp_line (start -9.525 -1.905) (end 4.445 -1.905) (stroke (width 0.12) (type solid)) (layer "F.SilkS"))
  (fp_line (start 4.445 12.065) (end -9.525 12.065) (stroke (width 0.12) (type solid)) (layer "F.SilkS"))
  (fp_line (start -9.525 12.065) (end -9.525 -1.905) (stroke (width 0.12) (type solid)) (layer "F.SilkS"))
  (pad "" np_thru_hole circle (at -7.62 5.08 90) (size 1.7 1.7) (drill 1.7) (layers "*.Cu" "*.Mask"))
  (pad "" np_thru_hole circle (at -2.54 5.08 90) (size 4 4) (drill 4) (layers "*.Cu" "*.Mask"))
  (pad "" np_thru_hole circle (at 2.54 5.08 90) (size 1.7 1.7) (drill 1.7) (layers "*.Cu" "*.Mask"))
  (pad "1" thru_hole circle (at 0 0 90) (size 2.2 2.2) (drill 1.5) (layers "*.Cu" "*.Mask") (remove_unused_layers no) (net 13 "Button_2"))
  (pad "2" thru_hole circle (at -6.35 2.54 90) (size 2.2 2.2) (drill 1.5) (layers "*.Cu" "*.Mask") (remove_unused_layers no) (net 2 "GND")))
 (gr_line (start 250 64.5) (end 177 64.5) (stroke (width 0.05) (type default)) (layer "Edge.Cuts"))
 (gr_line (start 267.5 109.5) (end 267.5 92) (stroke (width 0.05) (type default)) (layer "Edge.Cuts"))
 (gr_arc (start 251.469514 64.5) (mid 252.832831 64.827674) (end 253.898345 65.739097) (stroke (width 0.05) (type default))
  (layer "Edge.Cuts"))
 (gr_line (start 175 64.5) (end 177 64.5) (stroke (width 0.05) (type default)) (layer "Edge.Cuts"))
 (gr_line (start 185.601655 111.260903) (end 172.761558 93.550425) (stroke (width 0.05) (type default)) (layer "Edge.Cuts"))
 (gr_line (start 172 91.202555) (end 172 67.5) (stroke (width 0.05) (type default)) (layer "Edge.Cuts"))
 (gr_arc (start 172.761558 93.550425) (mid 172.195162 92.436699) (end 172 91.202555) (stroke (width 0.05) (type default))
  (layer "Edge.Cuts"))
 (gr_arc (start 267.5 109.5) (mid 266.62132 111.62132) (end 264.5 112.5) (stroke (width 0.05) (type default)) (layer "Edge.Cuts"))
 (gr_line (start 266.738442 83.449575) (end 253.898345 65.739097) (stroke (width 0.05) (type default)) (layer "Edge.Cuts"))
 (gr_line (start 251.469514 64.5) (end 250 64.5) (stroke (width 0.05) (type default)) (layer "Edge.Cuts"))
 (gr_line (start 267.5 92) (end 267.5 85.797445) (stroke (width 0.05) (type default)) (layer "Edge.Cuts"))
 (gr_line (start 188.030486 112.5) (end 264.5 112.5) (stroke (width 0.05) (type default)) (layer "Edge.Cuts"))
 (gr_arc (start 172 67.5) (mid 172.87868 65.37868) (end 175 64.5) (stroke (width 0.05) (type default)) (layer "Edge.Cuts"))
 (gr_arc (start 188.030486 112.5) (mid 186.667169 112.172326) (end 185.601655 111.260903) (stroke (width 0.05) (type default))
  (layer "Edge.Cuts"))
 (gr_arc (start 266.738442 83.449575) (mid 267.30485 84.563299) (end 267.5 85.797445) (stroke (width 0.05) (type default))
  (layer "Edge.Cuts"))
 (segment (start 209.059 94.711) (end 209.059 102.149) (width 0.2) (layer "F.Cu") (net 2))
 (segment (start 222.5 71.5) (end 228.56 71.5) (width 0.2) (layer "F.Cu") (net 2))
 (segment (start 208 74) (end 205.83 76.17) (width 0.2) (layer "F.Cu") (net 2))
 (segment (start 199.17 77) (end 200 76.17) (width 0.2) (layer "F.Cu") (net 2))
 (segment (start 214.27 89.5) (end 209.059 94.711) (width 0.2) (layer "F.Cu") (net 2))
 (segment (start 186.3 77) (end 199.17 77) (width 0.2) (layer "F.Cu") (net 2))
 (segment (start 232.46 106.09) (end 213 106.09) (width 0.2) (layer "F.Cu") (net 2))
 (segment (start 244.299528 105.231) (end 233.319 105.231) (width 0.2) (layer "F.Cu") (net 2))
 (segment (start 209.059 102.149) (end 213 106.09) (width 0.2) (layer "F.Cu") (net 2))
 (segment (start 193.71 106.09) (end 213 106.09) (width 0.2) (layer "F.Cu") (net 2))
 (segment (start 205.83 76.17) (end 200 76.17) (width 0.2) (layer "F.Cu") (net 2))
 (segment (start 233.319 105.231) (end 232.46 106.09) (width 0.2) (layer "F.Cu") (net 2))
 (segment (start 228.56 71.5) (end 233 75.94) (width 0.2) (layer "F.Cu") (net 2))
 (via (at 244.299528 105.231) (size 0.6) (drill 0.3) (layers "F.Cu" "B.Cu") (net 2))
 (segment (start 260.097 111.303) (end 252.68569 111.303) (width 0.2) (layer "B.Cu") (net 2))
 (segment (start 252.063 110.68031) (end 252.063 109.79969) (width 0.2) (layer "B.Cu") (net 2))
 (segment (start 261.16 110.24) (end 260.097 111.303) (width 0.2) (layer "B.Cu") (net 2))
 (segment (start 247.49431 105.231) (end 244.299528 105.231) (width 0.2) (layer "B.Cu") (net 2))
 (segment (start 252.063 109.79969) (end 247.49431 105.231) (width 0.2) (layer "B.Cu") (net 2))
 (segment (start 252.68569 111.303) (end 252.063 110.68031) (width 0.2) (layer "B.Cu") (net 2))
 (segment (start 210.5 71.5) (end 222.5 71.5) (width 0.2) (layer "B.Cu") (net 2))
 (segment (start 208 74) (end 210.5 71.5) (width 0.2) (layer "B.Cu") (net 2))
 (segment (start 251 110.24) (end 249.937 111.303) (width 0.2) (layer "B.Cu") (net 15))
 (segment (start 249.937 111.303) (end 213.003 111.303) (width 0.2) (layer "B.Cu") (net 15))
 (segment (start 213.003 111.303) (end 178.7 77) (width 0.2) (layer "B.Cu") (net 15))
 (segment (start 202.54 71.09) (end 200 73.63) (width 0.2) (layer "F.Cu") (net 3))
 (segment (start 202.54 70.4) (end 202.54 71.09) (width 0.2) (layer "F.Cu") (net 3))
 (segment (start 230.27 70.67) (end 233 73.4) (width 0.2) (layer "F.Cu") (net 1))
 (segment (start 230.27 70.17) (end 230.27 70.67) (width 0.2) (layer "F.Cu") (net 1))
 (segment (start 216.81 85.73) (end 216.81 89.5) (width 0.2) (layer "B.Cu") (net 10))
 (segment (start 218.04 84.5) (end 216.81 85.73) (width 0.2) (layer "B.Cu") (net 10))
 (segment (start 238.301 77.801) (end 199.214 77.801) (width 0.2) (layer "B.Cu") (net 12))
 (segment (start 197.46 76.047) (end 197.46 70.4) (width 0.2) (layer "B.Cu") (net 12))
 (segment (start 199.214 77.801) (end 197.46 76.047) (width 0.2) (layer "B.Cu") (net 12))
 (segment (start 255.5 95) (end 238.301 77.801) (width 0.2) (layer "B.Cu") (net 12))
 (segment (start 256.08 95) (end 255.5 95) (width 0.2) (layer "B.Cu") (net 12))
 (segment (start 253.54 88.36) (end 235.35 70.17) (width 0.2) (layer "F.Cu") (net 8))
 (segment (start 253.54 95) (end 253.54 88.36) (width 0.2) (layer "F.Cu") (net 8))
 (segment (start 213.961 85.501) (end 212.96 84.5) (width 0.2) (layer "F.Cu") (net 11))
 (segment (start 251 95) (end 251 94.386374) (width 0.2) (layer "F.Cu") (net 11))
 (segment (start 242.114626 85.501) (end 213.961 85.501) (width 0.2) (layer "F.Cu") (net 11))
 (segment (start 251 94.386374) (end 242.114626 85.501) (width 0.2) (layer "F.Cu") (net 11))
 (segment (start 191.17 105.531314) (end 191.17 99.74) (width 0.2) (layer "F.Cu") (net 7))
 (segment (start 263.7 95) (end 249.7 109) (width 0.2) (layer "F.Cu") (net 7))
 (segment (start 194.638686 109) (end 191.17 105.531314) (width 0.2) (layer "F.Cu") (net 7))
 (segment (start 249.7 109) (end 194.638686 109) (width 0.2) (layer "F.Cu") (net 7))
 (segment (start 232.829686 104.631) (end 251.529 104.631) (width 0.2) (layer "F.Cu") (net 13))
 (segment (start 227.938686 99.74) (end 232.829686 104.631) (width 0.2) (layer "F.Cu") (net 13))
 (segment (start 251.529 104.631) (end 261.16 95) (width 0.2) (layer "F.Cu") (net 13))
 (segment (start 210.46 99.74) (end 227.938686 99.74) (width 0.2) (layer "F.Cu") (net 13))
 (segment (start 229.92 99.74) (end 253.88 99.74) (width 0.2) (layer "F.Cu") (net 9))
 (segment (start 253.88 99.74) (end 258.62 95) (width 0.2) (layer "F.Cu") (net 9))
 (segment (start 218 78.718687) (end 210.781313 71.5) (width 0.2) (layer "F.Cu") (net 4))
 (segment (start 210.781313 71.5) (end 208 71.5) (width 0.2) (layer "F.Cu") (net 4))
 (segment (start 218 82) (end 218 78.718687) (width 0.2) (layer "F.Cu") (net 4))
 (via (at 218 82) (size 0.6) (drill 0.3) (layers "F.Cu" "B.Cu") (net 4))
 (segment (start 248.46 110.24) (end 238.149 99.929) (width 0.2) (layer "B.Cu") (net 4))
 (segment (start 235.929 99.929) (end 218 82) (width 0.2) (layer "B.Cu") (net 4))
 (segment (start 238.149 99.929) (end 235.929 99.929) (width 0.2) (layer "B.Cu") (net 4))
 (segment (start 257.544 94.39359) (end 237.88191 74.7315) (width 0.2) (layer "B.Cu") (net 5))
 (segment (start 237.88191 74.7315) (end 222.428608 74.7315) (width 0.2) (layer "B.Cu") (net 5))
 (segment (start 220.660108 76.5) (end 208 76.5) (width 0.2) (layer "B.Cu") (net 5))
 (segment (start 256.08 110.24) (end 257.544 108.776) (width 0.2) (layer "B.Cu") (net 5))
 (segment (start 257.544 108.776) (end 257.544 94.39359) (width 0.2) (layer "B.Cu") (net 5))
 (segment (start 222.428608 74.7315) (end 220.660108 76.5) (width 0.2) (layer "B.Cu") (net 5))
 (segment (start 223.4 77.4) (end 222.5 76.5) (width 0.2) (layer "B.Cu") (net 6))
 (segment (start 239.98331 77.4) (end 223.4 77.4) (width 0.2) (layer "B.Cu") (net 6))
 (segment (start 257.143 106.637) (end 257.143 94.55969) (width 0.2) (layer "B.Cu") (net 6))
 (segment (start 253.54 110.24) (end 257.143 106.637) (width 0.2) (layer "B.Cu") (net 6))
 (segment (start 257.143 94.55969) (end 239.98331 77.4) (width 0.2) (layer "B.Cu") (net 6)))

